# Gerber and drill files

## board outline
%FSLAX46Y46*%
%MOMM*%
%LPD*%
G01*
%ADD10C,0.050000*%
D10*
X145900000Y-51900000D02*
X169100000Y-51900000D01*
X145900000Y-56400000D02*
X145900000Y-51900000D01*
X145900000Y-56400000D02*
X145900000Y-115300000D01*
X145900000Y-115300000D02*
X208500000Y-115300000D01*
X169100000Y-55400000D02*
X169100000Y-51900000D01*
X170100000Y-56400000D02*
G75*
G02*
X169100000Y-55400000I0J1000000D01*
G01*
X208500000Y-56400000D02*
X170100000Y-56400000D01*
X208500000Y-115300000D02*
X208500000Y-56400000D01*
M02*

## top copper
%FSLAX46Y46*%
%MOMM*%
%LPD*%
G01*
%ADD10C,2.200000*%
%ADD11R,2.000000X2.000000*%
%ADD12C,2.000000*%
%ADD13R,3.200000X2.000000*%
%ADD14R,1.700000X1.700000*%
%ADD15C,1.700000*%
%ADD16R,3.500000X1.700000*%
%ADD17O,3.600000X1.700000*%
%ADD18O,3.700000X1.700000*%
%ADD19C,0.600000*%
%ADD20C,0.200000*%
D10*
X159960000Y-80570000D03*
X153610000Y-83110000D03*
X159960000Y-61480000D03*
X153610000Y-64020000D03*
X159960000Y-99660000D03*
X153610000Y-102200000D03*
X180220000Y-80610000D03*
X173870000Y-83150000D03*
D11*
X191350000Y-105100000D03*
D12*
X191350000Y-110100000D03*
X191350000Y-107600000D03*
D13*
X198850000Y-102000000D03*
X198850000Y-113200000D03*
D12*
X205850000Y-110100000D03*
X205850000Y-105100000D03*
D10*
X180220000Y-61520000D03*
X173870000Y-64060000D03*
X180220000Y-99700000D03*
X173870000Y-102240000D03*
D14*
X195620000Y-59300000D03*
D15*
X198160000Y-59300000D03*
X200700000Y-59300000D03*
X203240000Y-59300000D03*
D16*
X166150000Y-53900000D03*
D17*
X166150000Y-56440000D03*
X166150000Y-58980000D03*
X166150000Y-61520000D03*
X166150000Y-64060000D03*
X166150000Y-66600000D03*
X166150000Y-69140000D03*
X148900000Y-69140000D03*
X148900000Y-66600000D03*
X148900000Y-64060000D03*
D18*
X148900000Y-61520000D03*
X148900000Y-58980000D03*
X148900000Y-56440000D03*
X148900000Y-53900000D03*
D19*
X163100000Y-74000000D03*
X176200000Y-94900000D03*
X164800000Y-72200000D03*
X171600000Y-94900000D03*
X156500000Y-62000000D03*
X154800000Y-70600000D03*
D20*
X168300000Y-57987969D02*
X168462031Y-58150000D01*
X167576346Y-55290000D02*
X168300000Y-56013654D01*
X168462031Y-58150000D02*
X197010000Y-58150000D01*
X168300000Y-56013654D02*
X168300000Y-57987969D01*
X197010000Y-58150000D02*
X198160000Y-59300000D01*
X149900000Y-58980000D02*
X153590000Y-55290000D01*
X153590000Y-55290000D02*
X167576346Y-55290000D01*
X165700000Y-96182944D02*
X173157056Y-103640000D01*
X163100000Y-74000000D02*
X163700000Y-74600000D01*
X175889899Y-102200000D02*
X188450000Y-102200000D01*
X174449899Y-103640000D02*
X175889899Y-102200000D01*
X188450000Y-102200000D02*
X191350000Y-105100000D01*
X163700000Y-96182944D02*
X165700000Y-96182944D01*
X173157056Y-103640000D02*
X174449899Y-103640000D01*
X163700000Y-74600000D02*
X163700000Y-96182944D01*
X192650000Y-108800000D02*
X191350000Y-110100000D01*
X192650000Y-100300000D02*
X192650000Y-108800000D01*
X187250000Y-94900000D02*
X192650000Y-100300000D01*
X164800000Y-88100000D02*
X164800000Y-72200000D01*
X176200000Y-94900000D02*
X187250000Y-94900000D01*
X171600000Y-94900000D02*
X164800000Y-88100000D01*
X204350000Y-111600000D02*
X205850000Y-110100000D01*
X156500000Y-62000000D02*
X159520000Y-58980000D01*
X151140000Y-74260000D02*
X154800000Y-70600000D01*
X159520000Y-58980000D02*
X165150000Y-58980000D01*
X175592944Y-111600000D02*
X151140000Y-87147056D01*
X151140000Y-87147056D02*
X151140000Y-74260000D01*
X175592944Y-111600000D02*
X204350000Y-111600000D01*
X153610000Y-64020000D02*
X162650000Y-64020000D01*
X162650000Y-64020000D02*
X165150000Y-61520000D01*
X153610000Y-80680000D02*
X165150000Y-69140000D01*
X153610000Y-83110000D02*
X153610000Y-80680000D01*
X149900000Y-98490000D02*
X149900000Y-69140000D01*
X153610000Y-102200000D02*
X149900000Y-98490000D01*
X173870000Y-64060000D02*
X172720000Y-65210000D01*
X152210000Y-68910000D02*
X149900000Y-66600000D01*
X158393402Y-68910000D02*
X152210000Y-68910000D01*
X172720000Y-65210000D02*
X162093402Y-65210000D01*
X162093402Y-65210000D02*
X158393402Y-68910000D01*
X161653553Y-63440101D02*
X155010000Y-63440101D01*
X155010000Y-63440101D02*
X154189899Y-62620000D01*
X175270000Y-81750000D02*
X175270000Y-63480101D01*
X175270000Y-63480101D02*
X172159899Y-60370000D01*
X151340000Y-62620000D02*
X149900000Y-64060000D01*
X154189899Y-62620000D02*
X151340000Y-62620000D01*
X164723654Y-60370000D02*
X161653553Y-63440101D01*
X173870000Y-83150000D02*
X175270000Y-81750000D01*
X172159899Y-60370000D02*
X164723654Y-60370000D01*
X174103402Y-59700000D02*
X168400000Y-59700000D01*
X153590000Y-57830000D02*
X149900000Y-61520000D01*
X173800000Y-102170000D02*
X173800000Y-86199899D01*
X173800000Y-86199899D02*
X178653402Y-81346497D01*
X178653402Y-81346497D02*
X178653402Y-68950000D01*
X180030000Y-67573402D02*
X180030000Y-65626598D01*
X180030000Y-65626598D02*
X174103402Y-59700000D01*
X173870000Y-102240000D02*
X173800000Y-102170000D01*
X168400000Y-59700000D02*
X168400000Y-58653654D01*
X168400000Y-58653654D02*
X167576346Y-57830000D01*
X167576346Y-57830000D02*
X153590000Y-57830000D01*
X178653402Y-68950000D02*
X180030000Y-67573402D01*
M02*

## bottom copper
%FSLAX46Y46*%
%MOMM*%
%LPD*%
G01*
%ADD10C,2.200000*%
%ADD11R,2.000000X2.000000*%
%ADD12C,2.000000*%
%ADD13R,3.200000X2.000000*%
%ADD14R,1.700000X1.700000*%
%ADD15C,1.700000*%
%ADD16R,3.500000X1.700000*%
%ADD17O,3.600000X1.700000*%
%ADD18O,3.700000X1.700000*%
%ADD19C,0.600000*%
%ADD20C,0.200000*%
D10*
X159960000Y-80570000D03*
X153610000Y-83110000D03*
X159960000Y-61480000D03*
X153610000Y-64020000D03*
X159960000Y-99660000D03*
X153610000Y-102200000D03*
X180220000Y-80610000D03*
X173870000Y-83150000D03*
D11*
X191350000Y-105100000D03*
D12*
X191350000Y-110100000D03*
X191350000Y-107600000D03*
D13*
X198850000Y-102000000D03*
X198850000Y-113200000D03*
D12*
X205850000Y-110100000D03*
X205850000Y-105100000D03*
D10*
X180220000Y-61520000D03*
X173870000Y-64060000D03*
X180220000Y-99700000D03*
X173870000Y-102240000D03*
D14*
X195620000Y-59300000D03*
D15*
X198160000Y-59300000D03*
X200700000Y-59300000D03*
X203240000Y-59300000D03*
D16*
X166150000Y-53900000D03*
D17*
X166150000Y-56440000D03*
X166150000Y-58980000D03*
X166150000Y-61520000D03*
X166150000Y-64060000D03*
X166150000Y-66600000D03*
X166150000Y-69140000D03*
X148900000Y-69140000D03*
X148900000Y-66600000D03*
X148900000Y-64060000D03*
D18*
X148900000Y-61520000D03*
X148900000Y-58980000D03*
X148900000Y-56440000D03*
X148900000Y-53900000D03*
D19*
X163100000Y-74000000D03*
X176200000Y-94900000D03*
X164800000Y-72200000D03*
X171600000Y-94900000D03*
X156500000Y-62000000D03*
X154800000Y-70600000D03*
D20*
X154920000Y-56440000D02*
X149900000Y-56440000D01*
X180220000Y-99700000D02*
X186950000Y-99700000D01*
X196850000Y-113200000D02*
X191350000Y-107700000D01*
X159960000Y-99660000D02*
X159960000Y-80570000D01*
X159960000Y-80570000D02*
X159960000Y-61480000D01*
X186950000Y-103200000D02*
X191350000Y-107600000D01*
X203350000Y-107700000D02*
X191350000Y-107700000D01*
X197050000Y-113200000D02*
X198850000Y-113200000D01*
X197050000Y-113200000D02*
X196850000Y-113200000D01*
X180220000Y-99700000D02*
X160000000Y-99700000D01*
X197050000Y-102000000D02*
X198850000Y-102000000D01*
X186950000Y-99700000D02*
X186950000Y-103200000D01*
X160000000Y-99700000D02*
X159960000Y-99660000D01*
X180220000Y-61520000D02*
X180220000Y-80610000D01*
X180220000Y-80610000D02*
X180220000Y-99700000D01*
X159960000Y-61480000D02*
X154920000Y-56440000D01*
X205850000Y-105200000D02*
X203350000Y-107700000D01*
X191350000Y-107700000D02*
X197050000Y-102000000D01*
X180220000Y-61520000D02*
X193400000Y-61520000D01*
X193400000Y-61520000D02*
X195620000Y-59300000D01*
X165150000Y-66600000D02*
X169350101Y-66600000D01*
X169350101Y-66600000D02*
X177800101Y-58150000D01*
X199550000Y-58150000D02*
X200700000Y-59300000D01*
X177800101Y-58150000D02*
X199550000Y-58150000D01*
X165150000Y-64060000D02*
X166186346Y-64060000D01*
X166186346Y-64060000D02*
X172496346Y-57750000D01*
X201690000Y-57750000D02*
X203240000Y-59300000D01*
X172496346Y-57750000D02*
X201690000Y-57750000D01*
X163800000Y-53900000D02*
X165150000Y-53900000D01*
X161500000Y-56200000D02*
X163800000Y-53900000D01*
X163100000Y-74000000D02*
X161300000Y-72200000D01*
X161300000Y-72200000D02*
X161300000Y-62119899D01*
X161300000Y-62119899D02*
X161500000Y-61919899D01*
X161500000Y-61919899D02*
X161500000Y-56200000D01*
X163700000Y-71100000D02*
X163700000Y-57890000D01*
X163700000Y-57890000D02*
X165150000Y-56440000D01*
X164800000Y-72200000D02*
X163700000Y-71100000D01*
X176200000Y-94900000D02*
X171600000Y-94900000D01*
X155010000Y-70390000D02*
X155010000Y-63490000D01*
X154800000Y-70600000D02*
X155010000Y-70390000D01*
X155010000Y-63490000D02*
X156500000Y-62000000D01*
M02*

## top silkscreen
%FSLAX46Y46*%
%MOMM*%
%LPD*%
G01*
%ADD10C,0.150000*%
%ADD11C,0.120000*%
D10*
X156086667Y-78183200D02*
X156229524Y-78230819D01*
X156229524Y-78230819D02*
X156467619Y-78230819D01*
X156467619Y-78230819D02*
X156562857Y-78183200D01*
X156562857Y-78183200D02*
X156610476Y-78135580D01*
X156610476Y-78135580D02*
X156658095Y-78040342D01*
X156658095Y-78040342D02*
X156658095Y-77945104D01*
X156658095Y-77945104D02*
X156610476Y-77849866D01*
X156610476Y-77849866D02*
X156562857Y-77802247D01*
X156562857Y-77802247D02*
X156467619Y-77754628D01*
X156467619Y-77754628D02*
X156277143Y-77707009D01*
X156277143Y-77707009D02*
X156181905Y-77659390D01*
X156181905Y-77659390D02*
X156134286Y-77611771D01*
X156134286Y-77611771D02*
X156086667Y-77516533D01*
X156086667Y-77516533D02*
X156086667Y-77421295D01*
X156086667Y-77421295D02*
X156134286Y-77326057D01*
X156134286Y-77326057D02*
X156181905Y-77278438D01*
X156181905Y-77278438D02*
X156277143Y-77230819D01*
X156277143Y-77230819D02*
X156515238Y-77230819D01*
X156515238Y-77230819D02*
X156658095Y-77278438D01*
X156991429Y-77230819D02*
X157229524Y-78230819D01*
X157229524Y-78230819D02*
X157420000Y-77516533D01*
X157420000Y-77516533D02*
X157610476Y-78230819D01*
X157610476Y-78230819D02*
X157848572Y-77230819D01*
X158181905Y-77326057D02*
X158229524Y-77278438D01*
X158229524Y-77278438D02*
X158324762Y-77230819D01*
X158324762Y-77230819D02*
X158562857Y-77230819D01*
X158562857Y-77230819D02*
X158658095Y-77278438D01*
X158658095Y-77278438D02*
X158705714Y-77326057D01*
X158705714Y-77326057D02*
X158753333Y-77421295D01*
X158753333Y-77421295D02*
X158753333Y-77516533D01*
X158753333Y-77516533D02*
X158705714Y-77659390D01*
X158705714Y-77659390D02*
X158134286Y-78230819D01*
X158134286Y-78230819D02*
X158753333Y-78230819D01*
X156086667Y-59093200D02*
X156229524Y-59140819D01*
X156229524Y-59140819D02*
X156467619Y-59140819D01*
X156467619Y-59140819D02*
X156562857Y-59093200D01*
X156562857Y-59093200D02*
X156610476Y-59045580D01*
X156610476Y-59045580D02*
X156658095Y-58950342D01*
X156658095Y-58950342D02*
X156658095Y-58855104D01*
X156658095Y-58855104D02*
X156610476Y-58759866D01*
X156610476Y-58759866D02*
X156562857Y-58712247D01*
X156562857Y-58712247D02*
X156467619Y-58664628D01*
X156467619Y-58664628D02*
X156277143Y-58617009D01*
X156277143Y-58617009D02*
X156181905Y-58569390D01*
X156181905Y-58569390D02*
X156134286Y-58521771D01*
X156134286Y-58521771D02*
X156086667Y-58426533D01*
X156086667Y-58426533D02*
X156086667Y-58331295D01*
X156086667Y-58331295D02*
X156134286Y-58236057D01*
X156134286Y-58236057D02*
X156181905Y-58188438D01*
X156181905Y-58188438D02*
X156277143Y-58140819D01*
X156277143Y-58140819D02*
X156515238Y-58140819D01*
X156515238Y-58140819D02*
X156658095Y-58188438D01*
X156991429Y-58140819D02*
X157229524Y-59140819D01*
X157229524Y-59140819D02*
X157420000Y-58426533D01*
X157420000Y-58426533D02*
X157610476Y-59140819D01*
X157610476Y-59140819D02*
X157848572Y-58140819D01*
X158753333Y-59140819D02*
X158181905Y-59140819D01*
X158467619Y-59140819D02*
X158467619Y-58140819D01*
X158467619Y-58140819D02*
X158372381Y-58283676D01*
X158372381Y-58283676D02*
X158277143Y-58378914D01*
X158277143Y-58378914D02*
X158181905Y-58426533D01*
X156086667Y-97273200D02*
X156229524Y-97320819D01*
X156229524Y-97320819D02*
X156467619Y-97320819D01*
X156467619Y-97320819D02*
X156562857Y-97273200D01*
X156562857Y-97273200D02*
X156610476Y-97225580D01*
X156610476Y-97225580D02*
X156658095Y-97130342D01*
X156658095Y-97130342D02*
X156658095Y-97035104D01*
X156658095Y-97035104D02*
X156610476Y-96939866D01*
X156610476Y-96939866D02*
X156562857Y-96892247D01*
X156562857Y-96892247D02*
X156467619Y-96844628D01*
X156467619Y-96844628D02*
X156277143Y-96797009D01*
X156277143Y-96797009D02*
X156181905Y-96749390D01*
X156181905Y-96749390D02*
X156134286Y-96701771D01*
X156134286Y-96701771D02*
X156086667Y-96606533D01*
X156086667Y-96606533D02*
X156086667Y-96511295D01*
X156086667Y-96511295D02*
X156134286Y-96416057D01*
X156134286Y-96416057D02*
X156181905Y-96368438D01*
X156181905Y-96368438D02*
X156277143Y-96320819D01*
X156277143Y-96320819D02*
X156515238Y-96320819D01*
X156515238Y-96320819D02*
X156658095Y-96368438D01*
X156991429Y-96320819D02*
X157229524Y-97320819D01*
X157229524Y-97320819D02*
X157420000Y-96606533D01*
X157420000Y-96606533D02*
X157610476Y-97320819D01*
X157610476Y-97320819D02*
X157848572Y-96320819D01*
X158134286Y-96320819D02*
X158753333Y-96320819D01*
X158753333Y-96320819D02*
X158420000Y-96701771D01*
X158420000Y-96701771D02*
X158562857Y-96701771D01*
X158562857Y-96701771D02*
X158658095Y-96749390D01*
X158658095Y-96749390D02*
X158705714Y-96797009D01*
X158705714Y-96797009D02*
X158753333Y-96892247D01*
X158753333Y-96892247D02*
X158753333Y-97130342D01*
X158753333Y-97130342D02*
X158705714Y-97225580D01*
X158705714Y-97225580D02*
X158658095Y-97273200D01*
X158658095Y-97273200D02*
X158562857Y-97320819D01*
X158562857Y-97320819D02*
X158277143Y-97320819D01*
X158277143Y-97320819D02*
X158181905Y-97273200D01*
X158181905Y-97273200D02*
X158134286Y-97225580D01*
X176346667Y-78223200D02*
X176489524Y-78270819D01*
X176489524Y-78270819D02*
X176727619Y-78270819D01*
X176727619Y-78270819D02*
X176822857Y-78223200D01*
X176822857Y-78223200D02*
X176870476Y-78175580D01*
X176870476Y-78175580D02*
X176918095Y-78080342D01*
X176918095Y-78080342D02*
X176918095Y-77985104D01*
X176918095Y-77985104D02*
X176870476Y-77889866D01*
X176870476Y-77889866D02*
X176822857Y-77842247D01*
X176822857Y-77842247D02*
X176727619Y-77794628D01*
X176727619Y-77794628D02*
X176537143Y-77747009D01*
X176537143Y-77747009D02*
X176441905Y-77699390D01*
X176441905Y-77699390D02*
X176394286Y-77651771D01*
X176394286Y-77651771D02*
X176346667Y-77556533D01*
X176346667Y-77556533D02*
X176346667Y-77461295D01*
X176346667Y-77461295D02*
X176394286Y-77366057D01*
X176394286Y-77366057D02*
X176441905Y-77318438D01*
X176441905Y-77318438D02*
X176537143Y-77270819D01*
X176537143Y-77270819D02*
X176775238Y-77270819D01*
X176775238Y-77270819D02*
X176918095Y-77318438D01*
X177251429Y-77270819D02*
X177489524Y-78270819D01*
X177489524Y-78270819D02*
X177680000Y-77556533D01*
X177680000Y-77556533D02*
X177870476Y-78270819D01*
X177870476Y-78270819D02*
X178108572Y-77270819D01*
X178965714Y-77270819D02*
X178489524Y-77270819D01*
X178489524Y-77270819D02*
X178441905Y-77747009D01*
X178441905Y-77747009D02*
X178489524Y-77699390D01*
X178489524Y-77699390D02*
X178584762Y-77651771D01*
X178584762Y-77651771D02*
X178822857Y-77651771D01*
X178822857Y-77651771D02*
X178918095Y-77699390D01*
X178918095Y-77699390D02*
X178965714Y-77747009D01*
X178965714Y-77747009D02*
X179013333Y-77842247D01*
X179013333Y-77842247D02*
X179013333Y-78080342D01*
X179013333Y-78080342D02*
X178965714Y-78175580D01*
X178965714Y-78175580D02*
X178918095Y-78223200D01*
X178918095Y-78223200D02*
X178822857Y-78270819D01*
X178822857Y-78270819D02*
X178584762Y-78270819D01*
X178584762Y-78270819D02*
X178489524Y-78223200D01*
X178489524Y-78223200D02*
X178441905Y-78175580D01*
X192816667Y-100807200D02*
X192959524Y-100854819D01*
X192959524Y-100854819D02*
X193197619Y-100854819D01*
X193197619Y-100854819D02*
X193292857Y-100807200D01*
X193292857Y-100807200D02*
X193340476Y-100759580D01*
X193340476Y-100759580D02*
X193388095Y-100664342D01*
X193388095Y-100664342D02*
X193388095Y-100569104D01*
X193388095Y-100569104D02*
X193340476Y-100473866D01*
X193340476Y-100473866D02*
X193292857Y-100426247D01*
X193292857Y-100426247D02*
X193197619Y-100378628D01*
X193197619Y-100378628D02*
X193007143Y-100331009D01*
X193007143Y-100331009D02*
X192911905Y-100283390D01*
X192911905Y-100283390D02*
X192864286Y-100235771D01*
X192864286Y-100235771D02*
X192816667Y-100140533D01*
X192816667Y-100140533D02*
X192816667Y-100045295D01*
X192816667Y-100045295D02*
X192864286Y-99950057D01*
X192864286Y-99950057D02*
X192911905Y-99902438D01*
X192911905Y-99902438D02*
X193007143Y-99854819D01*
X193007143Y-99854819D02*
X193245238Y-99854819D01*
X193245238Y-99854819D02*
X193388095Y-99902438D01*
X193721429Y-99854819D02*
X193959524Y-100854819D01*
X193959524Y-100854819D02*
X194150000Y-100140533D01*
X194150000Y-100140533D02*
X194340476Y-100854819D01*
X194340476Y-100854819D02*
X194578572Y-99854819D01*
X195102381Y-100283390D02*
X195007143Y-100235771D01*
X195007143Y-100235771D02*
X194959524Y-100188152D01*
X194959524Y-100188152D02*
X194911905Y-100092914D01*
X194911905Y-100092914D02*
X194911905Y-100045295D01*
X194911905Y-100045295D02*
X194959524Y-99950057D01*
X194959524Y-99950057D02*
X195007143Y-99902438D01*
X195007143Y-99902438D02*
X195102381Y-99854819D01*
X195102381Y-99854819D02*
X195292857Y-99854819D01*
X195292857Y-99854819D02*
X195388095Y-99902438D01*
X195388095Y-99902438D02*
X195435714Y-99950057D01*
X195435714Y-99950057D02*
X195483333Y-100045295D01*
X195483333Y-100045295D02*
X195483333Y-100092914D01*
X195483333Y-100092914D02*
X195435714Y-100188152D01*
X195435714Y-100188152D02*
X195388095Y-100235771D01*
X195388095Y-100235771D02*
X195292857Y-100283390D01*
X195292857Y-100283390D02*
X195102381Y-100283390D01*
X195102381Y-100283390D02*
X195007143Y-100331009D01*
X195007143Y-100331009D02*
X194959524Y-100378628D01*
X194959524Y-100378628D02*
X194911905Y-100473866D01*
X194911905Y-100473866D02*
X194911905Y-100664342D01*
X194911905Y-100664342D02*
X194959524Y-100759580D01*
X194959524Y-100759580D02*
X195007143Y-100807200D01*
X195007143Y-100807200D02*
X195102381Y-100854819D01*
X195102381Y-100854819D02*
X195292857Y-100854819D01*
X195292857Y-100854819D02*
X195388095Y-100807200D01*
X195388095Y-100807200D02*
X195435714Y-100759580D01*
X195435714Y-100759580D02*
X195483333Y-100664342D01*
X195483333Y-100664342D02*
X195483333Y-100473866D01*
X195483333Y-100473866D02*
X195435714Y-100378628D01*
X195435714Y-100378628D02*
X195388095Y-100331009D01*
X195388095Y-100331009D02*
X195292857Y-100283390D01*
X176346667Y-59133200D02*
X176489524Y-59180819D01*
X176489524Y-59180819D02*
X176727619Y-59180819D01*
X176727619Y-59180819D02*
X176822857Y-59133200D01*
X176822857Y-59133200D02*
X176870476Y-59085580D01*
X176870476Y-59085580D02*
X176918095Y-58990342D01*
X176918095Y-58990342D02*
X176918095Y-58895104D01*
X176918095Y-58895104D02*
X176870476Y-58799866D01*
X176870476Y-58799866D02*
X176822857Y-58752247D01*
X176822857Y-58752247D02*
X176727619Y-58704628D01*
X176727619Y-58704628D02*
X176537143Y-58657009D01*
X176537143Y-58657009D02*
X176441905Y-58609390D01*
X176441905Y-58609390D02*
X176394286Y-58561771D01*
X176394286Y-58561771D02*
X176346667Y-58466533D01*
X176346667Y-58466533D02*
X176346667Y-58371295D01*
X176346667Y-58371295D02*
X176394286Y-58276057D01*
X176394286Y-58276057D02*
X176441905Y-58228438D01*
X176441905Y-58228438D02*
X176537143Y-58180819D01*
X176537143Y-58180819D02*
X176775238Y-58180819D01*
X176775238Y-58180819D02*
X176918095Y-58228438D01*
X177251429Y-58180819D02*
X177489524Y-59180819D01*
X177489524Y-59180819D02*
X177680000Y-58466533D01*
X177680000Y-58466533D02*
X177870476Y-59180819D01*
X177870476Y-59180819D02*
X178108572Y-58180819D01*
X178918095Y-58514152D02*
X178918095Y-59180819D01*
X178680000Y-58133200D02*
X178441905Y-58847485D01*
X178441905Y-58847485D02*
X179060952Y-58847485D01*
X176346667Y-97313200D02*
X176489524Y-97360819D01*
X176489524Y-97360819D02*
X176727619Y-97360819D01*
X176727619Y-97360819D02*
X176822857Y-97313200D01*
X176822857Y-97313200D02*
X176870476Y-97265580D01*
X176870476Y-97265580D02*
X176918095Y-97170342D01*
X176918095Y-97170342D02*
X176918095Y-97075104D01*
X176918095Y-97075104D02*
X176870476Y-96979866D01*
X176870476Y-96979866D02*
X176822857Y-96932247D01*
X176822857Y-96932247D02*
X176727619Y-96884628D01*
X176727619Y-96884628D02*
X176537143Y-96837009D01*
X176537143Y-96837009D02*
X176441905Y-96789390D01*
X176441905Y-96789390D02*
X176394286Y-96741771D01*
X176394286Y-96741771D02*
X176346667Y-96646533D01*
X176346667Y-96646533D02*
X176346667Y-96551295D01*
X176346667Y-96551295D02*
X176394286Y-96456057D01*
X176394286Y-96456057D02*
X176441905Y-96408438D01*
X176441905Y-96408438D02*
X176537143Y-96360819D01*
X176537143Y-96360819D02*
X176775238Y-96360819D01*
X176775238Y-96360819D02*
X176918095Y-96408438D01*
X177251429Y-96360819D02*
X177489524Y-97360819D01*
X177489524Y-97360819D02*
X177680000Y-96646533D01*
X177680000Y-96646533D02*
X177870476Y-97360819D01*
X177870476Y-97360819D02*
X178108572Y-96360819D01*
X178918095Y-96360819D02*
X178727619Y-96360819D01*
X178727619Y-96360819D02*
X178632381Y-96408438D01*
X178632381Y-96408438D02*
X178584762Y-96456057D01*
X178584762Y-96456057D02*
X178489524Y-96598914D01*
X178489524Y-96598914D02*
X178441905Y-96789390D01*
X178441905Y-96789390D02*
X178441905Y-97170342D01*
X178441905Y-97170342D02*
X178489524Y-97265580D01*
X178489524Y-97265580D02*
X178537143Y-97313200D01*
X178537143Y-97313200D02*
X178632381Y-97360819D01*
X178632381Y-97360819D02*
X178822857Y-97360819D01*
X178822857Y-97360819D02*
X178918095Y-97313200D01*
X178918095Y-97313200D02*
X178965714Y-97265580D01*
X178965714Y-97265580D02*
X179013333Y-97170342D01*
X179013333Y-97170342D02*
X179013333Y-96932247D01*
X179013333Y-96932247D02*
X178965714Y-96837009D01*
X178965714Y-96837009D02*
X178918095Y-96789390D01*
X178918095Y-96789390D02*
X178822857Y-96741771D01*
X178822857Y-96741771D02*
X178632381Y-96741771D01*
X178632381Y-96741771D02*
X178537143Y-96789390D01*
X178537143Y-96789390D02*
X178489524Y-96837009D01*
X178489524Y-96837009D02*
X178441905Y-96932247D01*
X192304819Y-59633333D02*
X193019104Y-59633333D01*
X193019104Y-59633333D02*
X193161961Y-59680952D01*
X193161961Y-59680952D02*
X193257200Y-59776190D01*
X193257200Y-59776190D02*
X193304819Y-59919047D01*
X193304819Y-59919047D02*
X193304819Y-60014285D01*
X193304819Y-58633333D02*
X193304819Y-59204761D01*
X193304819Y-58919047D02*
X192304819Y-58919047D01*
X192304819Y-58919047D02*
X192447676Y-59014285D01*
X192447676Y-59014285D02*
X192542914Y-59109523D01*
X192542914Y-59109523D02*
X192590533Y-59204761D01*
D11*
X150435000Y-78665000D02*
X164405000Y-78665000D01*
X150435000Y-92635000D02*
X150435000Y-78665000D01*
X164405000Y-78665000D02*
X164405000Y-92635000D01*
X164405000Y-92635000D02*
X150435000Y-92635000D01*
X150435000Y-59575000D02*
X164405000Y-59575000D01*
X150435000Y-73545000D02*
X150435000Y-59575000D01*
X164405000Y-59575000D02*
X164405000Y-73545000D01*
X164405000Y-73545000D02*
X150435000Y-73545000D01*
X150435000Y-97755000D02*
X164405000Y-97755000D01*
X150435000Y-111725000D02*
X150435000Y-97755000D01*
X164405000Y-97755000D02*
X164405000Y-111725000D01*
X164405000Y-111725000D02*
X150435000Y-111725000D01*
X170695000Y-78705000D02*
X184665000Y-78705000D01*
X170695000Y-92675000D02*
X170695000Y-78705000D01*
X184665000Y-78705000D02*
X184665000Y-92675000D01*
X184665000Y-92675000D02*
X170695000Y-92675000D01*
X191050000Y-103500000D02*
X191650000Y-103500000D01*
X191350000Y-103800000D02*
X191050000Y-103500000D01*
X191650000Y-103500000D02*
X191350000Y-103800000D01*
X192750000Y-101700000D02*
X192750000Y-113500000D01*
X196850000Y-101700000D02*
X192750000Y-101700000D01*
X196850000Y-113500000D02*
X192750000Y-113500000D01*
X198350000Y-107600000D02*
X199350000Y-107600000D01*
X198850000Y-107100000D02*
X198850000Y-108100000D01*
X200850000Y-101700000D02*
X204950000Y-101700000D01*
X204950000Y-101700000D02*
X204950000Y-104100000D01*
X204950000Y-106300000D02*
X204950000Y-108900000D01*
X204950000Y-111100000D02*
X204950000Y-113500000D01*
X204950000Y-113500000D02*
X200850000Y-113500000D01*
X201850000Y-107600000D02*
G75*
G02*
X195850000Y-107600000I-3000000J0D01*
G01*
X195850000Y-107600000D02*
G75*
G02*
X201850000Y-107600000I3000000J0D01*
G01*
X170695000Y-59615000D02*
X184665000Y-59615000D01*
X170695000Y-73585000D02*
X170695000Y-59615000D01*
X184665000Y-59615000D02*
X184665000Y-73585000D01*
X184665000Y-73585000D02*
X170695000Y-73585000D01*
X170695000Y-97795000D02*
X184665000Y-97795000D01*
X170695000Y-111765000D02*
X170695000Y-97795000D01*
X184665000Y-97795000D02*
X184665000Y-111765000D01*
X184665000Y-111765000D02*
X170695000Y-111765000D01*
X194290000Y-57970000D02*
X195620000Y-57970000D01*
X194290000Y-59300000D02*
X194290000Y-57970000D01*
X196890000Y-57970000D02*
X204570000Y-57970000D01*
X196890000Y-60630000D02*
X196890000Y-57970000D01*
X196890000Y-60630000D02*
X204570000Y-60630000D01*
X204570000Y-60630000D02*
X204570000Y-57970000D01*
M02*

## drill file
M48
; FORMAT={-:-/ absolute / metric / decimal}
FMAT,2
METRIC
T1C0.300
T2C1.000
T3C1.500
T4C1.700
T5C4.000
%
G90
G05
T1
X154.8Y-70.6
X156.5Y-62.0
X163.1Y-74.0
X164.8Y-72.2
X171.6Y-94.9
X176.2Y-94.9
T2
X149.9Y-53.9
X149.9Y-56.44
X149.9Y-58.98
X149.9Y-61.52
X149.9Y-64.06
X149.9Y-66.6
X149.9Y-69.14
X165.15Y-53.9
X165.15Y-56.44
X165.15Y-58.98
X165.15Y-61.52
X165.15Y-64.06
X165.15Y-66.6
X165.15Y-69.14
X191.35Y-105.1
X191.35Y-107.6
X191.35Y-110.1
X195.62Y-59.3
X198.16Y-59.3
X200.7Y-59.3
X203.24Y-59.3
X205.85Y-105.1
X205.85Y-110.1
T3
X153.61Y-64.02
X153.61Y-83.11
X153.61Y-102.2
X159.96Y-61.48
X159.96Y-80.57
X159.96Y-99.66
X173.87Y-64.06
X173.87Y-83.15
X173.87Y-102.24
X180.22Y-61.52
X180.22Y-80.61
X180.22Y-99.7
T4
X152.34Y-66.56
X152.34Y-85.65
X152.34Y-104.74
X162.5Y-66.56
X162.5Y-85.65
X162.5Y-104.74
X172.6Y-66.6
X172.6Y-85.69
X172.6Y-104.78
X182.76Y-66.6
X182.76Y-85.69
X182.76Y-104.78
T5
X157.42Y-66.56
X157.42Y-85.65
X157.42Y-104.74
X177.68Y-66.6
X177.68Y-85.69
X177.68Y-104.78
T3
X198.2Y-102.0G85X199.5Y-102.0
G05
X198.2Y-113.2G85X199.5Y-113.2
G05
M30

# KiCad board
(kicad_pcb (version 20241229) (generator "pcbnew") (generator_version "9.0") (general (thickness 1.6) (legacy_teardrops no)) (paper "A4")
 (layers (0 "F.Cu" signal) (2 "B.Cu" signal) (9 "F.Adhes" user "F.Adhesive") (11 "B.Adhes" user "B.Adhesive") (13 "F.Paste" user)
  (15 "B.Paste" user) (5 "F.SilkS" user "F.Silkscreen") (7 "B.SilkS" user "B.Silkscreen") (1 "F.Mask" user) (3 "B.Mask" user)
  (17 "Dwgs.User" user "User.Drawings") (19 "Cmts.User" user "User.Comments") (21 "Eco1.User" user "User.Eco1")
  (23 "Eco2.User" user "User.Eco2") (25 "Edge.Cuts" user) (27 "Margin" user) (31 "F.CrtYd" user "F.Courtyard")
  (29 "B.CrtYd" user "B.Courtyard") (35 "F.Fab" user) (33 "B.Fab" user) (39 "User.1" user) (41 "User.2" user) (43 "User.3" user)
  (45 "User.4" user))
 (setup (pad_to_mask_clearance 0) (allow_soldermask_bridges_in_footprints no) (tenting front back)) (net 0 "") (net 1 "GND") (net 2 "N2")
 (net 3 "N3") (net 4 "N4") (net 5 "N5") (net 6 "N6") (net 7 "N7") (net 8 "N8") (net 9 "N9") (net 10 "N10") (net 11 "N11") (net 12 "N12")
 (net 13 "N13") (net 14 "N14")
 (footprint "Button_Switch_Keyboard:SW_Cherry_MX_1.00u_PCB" (layer "F.Cu") (at 159.96 80.57)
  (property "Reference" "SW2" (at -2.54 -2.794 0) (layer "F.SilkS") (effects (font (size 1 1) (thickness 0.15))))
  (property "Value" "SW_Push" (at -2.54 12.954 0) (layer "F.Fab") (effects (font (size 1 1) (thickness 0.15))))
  (fp_line (start -9.525 -1.905) (end 4.445 -1.905) (stroke (width 0.12) (type solid)) (layer "F.SilkS"))
  (fp_line (start -9.525 12.065) (end -9.525 -1.905) (stroke (width 0.12) (type solid)) (layer "F.SilkS"))
  (fp_line (start 4.445 -1.905) (end 4.445 12.065) (stroke (width 0.12) (type solid)) (layer "F.SilkS"))
  (fp_line (start 4.445 12.065) (end -9.525 12.065) (stroke (width 0.12) (type solid)) (layer "F.SilkS"))
  (pad "" np_thru_hole circle (at -7.62 5.08) (size 1.7 1.7) (drill 1.7) (layers "*.Cu" "*.Mask"))
  (pad "" np_thru_hole circle (at -2.54 5.08) (size 4 4) (drill 4) (layers "*.Cu" "*.Mask"))
  (pad "" np_thru_hole circle (at 2.54 5.08) (size 1.7 1.7) (drill 1.7) (layers "*.Cu" "*.Mask"))
  (pad "1" thru_hole circle (at 0 0) (size 2.2 2.2) (drill 1.5) (layers "*.Cu" "*.Mask") (remove_unused_layers no) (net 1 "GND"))
  (pad "2" thru_hole circle (at -6.35 2.54) (size 2.2 2.2) (drill 1.5) (layers "*.Cu" "*.Mask") (remove_unused_layers no) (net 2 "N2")))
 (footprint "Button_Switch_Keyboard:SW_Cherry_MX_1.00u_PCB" (layer "F.Cu") (at 159.96 61.48)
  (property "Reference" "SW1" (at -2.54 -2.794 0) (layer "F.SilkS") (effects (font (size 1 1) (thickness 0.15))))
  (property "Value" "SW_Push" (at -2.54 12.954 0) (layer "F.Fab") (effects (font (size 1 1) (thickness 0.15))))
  (fp_line (start -9.525 -1.905) (end 4.445 -1.905) (stroke (width 0.12) (type solid)) (layer "F.SilkS"))
  (fp_line (start -9.525 12.065) (end -9.525 -1.905) (stroke (width 0.12) (type solid)) (layer "F.SilkS"))
  (fp_line (start 4.445 -1.905) (end 4.445 12.065) (stroke (width 0.12) (type solid)) (layer "F.SilkS"))
  (fp_line (start 4.445 12.065) (end -9.525 12.065) (stroke (width 0.12) (type solid)) (layer "F.SilkS"))
  (pad "" np_thru_hole circle (at -7.62 5.08) (size 1.7 1.7) (drill 1.7) (layers "*.Cu" "*.Mask"))
  (pad "" np_thru_hole circle (at -2.54 5.08) (size 4 4) (drill 4) (layers "*.Cu" "*.Mask"))
  (pad "" np_thru_hole circle (at 2.54 5.08) (size 1.7 1.7) (drill 1.7) (layers "*.Cu" "*.Mask"))
  (pad "1" thru_hole circle (at 0 0) (size 2.2 2.2) (drill 1.5) (layers "*.Cu" "*.Mask") (remove_unused_layers no) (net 1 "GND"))
  (pad "2" thru_hole circle (at -6.35 2.54) (size 2.2 2.2) (drill 1.5) (layers "*.Cu" "*.Mask") (remove_unused_layers no) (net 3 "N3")))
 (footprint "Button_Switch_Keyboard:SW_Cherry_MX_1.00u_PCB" (layer "F.Cu") (at 159.96 99.66)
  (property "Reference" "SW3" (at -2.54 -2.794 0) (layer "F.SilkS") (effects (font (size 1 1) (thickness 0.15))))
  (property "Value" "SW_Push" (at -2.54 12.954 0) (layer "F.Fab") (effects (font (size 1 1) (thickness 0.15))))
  (fp_line (start -9.525 -1.905) (end 4.445 -1.905) (stroke (width 0.12) (type solid)) (layer "F.SilkS"))
  (fp_line (start -9.525 12.065) (end -9.525 -1.905) (stroke (width 0.12) (type solid)) (layer "F.SilkS"))
  (fp_line (start 4.445 -1.905) (end 4.445 12.065) (stroke (width 0.12) (type solid)) (layer "F.SilkS"))
  (fp_line (start 4.445 12.065) (end -9.525 12.065) (stroke (width 0.12) (type solid)) (layer "F.SilkS"))
  (pad "" np_thru_hole circle (at -7.62 5.08) (size 1.7 1.7) (drill 1.7) (layers "*.Cu" "*.Mask"))
  (pad "" np_thru_hole circle (at -2.54 5.08) (size 4 4) (drill 4) (layers "*.Cu" "*.Mask"))
  (pad "" np_thru_hole circle (at 2.54 5.08) (size 1.7 1.7) (drill 1.7) (layers "*.Cu" "*.Mask"))
  (pad "1" thru_hole circle (at 0 0) (size 2.2 2.2) (drill 1.5) (layers "*.Cu" "*.Mask") (remove_unused_layers no) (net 1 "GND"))
  (pad "2" thru_hole circle (at -6.35 2.54) (size 2.2 2.2) (drill 1.5) (layers "*.Cu" "*.Mask") (remove_unused_layers no) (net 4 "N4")))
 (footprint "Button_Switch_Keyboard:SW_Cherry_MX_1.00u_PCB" (layer "F.Cu") (at 180.22 80.61)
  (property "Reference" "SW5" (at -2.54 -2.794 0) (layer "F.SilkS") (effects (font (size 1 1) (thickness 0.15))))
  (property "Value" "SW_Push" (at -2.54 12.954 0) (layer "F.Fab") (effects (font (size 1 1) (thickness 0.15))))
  (fp_line (start -9.525 -1.905) (end 4.445 -1.905) (stroke (width 0.12) (type solid)) (layer "F.SilkS"))
  (fp_line (start -9.525 12.065) (end -9.525 -1.905) (stroke (width 0.12) (type solid)) (layer "F.SilkS"))
  (fp_line (start 4.445 -1.905) (end 4.445 12.065) (stroke (width 0.12) (type solid)) (layer "F.SilkS"))
  (fp_line (start 4.445 12.065) (end -9.525 12.065) (stroke (width 0.12) (type solid)) (layer "F.SilkS"))
  (pad "" np_thru_hole circle (at -7.62 5.08) (size 1.7 1.7) (drill 1.7) (layers "*.Cu" "*.Mask"))
  (pad "" np_thru_hole circle (at -2.54 5.08) (size 4 4) (drill 4) (layers "*.Cu" "*.Mask"))
  (pad "" np_thru_hole circle (at 2.54 5.08) (size 1.7 1.7) (drill 1.7) (layers "*.Cu" "*.Mask"))
  (pad "1" thru_hole circle (at 0 0) (size 2.2 2.2) (drill 1.5) (layers "*.Cu" "*.Mask") (remove_unused_layers no) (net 1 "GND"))
  (pad "2" thru_hole circle (at -6.35 2.54) (size 2.2 2.2) (drill 1.5) (layers "*.Cu" "*.Mask") (remove_unused_layers no) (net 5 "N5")))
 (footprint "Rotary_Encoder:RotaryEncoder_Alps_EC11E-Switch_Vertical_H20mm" (layer "F.Cu") (at 191.35 105.1)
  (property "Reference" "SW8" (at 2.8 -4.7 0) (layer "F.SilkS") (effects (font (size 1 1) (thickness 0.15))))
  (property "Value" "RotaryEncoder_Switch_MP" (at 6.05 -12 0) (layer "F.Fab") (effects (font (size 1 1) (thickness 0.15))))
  (fp_line (start -0.3 -1.6) (end 0.3 -1.6) (stroke (width 0.12) (type solid)) (layer "F.SilkS"))
  (fp_line (start 0 -1.3) (end -0.3 -1.6) (stroke (width 0.12) (type solid)) (layer "F.SilkS"))
  (fp_line (start 0.3 -1.6) (end 0 -1.3) (stroke (width 0.12) (type solid)) (layer "F.SilkS"))
  (fp_line (start 1.4 -3.4) (end 1.4 8.4) (stroke (width 0.12) (type solid)) (layer "F.SilkS"))
  (fp_line (start 5.5 -3.4) (end 1.4 -3.4) (stroke (width 0.12) (type solid)) (layer "F.SilkS"))
  (fp_line (start 5.5 8.4) (end 1.4 8.4) (stroke (width 0.12) (type solid)) (layer "F.SilkS"))
  (fp_line (start 7 2.5) (end 8 2.5) (stroke (width 0.12) (type solid)) (layer "F.SilkS"))
  (fp_line (start 7.5 2) (end 7.5 3) (stroke (width 0.12) (type solid)) (layer "F.SilkS"))
  (fp_line (start 9.5 -3.4) (end 13.6 -3.4) (stroke (width 0.12) (type solid)) (layer "F.SilkS"))
  (fp_line (start 13.6 -3.4) (end 13.6 -1) (stroke (width 0.12) (type solid)) (layer "F.SilkS"))
  (fp_line (start 13.6 1.2) (end 13.6 3.8) (stroke (width 0.12) (type solid)) (layer "F.SilkS"))
  (fp_line (start 13.6 6) (end 13.6 8.4) (stroke (width 0.12) (type solid)) (layer "F.SilkS"))
  (fp_line (start 13.6 8.4) (end 9.5 8.4) (stroke (width 0.12) (type solid)) (layer "F.SilkS"))
  (fp_circle (center 7.5 2.5) (end 10.5 2.5) (stroke (width 0.12) (type solid)) (fill no) (layer "F.SilkS"))
  (pad "A" thru_hole rect (at 0 0) (size 2 2) (drill 1) (layers "*.Cu" "*.Mask") (remove_unused_layers no) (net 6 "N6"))
  (pad "B" thru_hole circle (at 0 5) (size 2 2) (drill 1) (layers "*.Cu" "*.Mask") (remove_unused_layers no) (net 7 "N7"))
  (pad "C" thru_hole circle (at 0 2.5) (size 2 2) (drill 1) (layers "*.Cu" "*.Mask") (remove_unused_layers no) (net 1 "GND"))
  (pad "MP" thru_hole rect (at 7.5 -3.1) (size 3.2 2) (drill oval 2.8 1.5) (layers "*.Cu" "*.Mask") (remove_unused_layers no) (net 1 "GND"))
  (pad "MP" thru_hole rect (at 7.5 8.1) (size 3.2 2) (drill oval 2.8 1.5) (layers "*.Cu" "*.Mask") (remove_unused_layers no) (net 1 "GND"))
  (pad "S1" thru_hole circle (at 14.5 5) (size 2 2) (drill 1) (layers "*.Cu" "*.Mask") (remove_unused_layers no) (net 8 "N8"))
  (pad "S2" thru_hole circle (at 14.5 0) (size 2 2) (drill 1) (layers "*.Cu" "*.Mask") (remove_unused_layers no) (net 1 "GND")))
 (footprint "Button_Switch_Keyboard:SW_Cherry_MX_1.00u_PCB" (layer "F.Cu") (at 180.22 61.52)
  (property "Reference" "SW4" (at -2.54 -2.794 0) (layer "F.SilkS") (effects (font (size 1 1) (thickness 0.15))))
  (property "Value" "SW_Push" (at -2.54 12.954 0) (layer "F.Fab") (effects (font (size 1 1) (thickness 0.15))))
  (fp_line (start -9.525 -1.905) (end 4.445 -1.905) (stroke (width 0.12) (type solid)) (layer "F.SilkS"))
  (fp_line (start -9.525 12.065) (end -9.525 -1.905) (stroke (width 0.12) (type solid)) (layer "F.SilkS"))
  (fp_line (start 4.445 -1.905) (end 4.445 12.065) (stroke (width 0.12) (type solid)) (layer "F.SilkS"))
  (fp_line (start 4.445 12.065) (end -9.525 12.065) (stroke (width 0.12) (type solid)) (layer "F.SilkS"))
  (pad "" np_thru_hole circle (at -7.62 5.08) (size 1.7 1.7) (drill 1.7) (layers "*.Cu" "*.Mask"))
  (pad "" np_thru_hole circle (at -2.54 5.08) (size 4 4) (drill 4) (layers "*.Cu" "*.Mask"))
  (pad "" np_thru_hole circle (at 2.54 5.08) (size 1.7 1.7) (drill 1.7) (layers "*.Cu" "*.Mask"))
  (pad "1" thru_hole circle (at 0 0) (size 2.2 2.2) (drill 1.5) (layers "*.Cu" "*.Mask") (remove_unused_layers no) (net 1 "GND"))
  (pad "2" thru_hole circle (at -6.35 2.54) (size 2.2 2.2) (drill 1.5) (layers "*.Cu" "*.Mask") (remove_unused_layers no) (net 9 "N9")))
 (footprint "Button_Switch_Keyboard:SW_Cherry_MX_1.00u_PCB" (layer "F.Cu") (at 180.22 99.7)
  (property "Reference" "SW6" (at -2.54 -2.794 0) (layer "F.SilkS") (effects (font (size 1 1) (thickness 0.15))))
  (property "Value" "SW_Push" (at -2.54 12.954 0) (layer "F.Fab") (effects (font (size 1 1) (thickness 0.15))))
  (fp_line (start -9.525 -1.905) (end 4.445 -1.905) (stroke (width 0.12) (type solid)) (layer "F.SilkS"))
  (fp_line (start -9.525 12.065) (end -9.525 -1.905) (stroke (width 0.12) (type solid)) (layer "F.SilkS"))
  (fp_line (start 4.445 -1.905) (end 4.445 12.065) (stroke (width 0.12) (type solid)) (layer "F.SilkS"))
  (fp_line (start 4.445 12.065) (end -9.525 12.065) (stroke (width 0.12) (type solid)) (layer "F.SilkS"))
  (pad "" np_thru_hole circle (at -7.62 5.08) (size 1.7 1.7) (drill 1.7) (layers "*.Cu" "*.Mask"))
  (pad "" np_thru_hole circle (at -2.54 5.08) (size 4 4) (drill 4) (layers "*.Cu" "*.Mask"))
  (pad "" np_thru_hole circle (at 2.54 5.08) (size 1.7 1.7) (drill 1.7) (layers "*.Cu" "*.Mask"))
  (pad "1" thru_hole circle (at 0 0) (size 2.2 2.2) (drill 1.5) (layers "*.Cu" "*.Mask") (remove_unused_layers no) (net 1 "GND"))
  (pad "2" thru_hole circle (at -6.35 2.54) (size 2.2 2.2) (drill 1.5) (layers "*.Cu" "*.Mask") (remove_unused_layers no) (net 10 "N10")))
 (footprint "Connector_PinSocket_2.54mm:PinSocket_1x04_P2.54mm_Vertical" (layer "F.Cu") (at 195.62 59.3 90)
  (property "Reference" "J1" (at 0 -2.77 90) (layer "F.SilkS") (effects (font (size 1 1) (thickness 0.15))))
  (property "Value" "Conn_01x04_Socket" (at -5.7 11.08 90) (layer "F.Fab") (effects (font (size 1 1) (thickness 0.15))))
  (fp_line (start 1.33 -1.33) (end 1.33 0) (stroke (width 0.12) (type solid)) (layer "F.SilkS"))
  (fp_line (start 0 -1.33) (end 1.33 -1.33) (stroke (width 0.12) (type solid)) (layer "F.SilkS"))
  (fp_line (start 1.33 1.27) (end 1.33 8.95) (stroke (width 0.12) (type solid)) (layer "F.SilkS"))
  (fp_line (start -1.33 1.27) (end 1.33 1.27) (stroke (width 0.12) (type solid)) (layer "F.SilkS"))
  (fp_line (start -1.33 1.27) (end -1.33 8.95) (stroke (width 0.12) (type solid)) (layer "F.SilkS"))
  (fp_line (start -1.33 8.95) (end 1.33 8.95) (stroke (width 0.12) (type solid)) (layer "F.SilkS"))
  (pad "1" thru_hole rect (at 0 0 90) (size 1.7 1.7) (drill 1) (layers "*.Cu" "*.Mask") (remove_unused_layers no) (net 1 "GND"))
  (pad "2" thru_hole circle (at 0 2.54 90) (size 1.7 1.7) (drill 1) (layers "*.Cu" "*.Mask") (remove_unused_layers no) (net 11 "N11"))
  (pad "3" thru_hole circle (at 0 5.08 90) (size 1.7 1.7) (drill 1) (layers "*.Cu" "*.Mask") (remove_unused_layers no) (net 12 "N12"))
  (pad "4" thru_hole circle (at 0 7.62 90) (size 1.7 1.7) (drill 1) (layers "*.Cu" "*.Mask") (remove_unused_layers no) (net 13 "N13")))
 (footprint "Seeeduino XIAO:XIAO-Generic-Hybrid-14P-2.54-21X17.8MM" (layer "B.Cu") (at 157.525 61.52 180)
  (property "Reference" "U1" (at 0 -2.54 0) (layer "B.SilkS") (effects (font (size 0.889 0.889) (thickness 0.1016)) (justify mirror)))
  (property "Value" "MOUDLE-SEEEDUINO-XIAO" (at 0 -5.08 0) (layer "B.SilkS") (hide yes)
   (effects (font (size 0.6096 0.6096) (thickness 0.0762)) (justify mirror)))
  (pad "1" thru_hole rect (at -7.625 7.62 180) (size 3.5 1.7) (drill 1 (offset -1 0)) (layers "*.Cu" "*.Mask") (remove_unused_layers no)
   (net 6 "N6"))
  (pad "2" thru_hole oval (at -7.625 5.08 180) (size 3.6 1.7) (drill 1 (offset -1 0)) (layers "*.Cu" "*.Mask") (remove_unused_layers no)
   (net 7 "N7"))
  (pad "3" thru_hole oval (at -7.625 2.54 180) (size 3.6 1.7) (drill 1 (offset -1 0)) (layers "*.Cu" "*.Mask") (remove_unused_layers no)
   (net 8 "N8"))
  (pad "4" thru_hole oval (at -7.625 0 180) (size 3.6 1.7) (drill 1 (offset -1 0)) (layers "*.Cu" "*.Mask") (remove_unused_layers no)
   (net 3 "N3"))
  (pad "5" thru_hole oval (at -7.625 -2.54 180) (size 3.6 1.7) (drill 1 (offset -1 0)) (layers "*.Cu" "*.Mask") (remove_unused_layers no)
   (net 13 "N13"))
  (pad "6" thru_hole oval (at -7.625 -5.08) (size 3.6 1.7) (drill 1 (offset 1 0)) (layers "*.Cu" "*.Mask") (remove_unused_layers no)
   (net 12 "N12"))
  (pad "7" thru_hole oval (at -7.625 -7.62 180) (size 3.6 1.7) (drill 1 (offset -1 0)) (layers "*.Cu" "*.Mask") (remove_unused_layers no)
   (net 2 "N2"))
  (pad "8" thru_hole oval (at 7.625 -7.62 180) (size 3.6 1.7) (drill 1 (offset 1 0)) (layers "*.Cu" "*.Mask") (remove_unused_layers no)
   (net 4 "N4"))
  (pad "9" thru_hole oval (at 7.625 -5.08 180) (size 3.6 1.7) (drill 1 (offset 1 0)) (layers "*.Cu" "*.Mask") (remove_unused_layers no)
   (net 9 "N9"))
  (pad "10" thru_hole oval (at 7.625 -2.54 180) (size 3.6 1.7) (drill 1 (offset 1 0)) (layers "*.Cu" "*.Mask") (remove_unused_layers no)
   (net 5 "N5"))
  (pad "11" thru_hole oval (at 7.625 0 180) (size 3.7 1.7) (drill 1 (offset 1 0)) (layers "*.Cu" "*.Mask") (remove_unused_layers no)
   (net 10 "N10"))
  (pad "12" thru_hole oval (at 7.625 2.54 180) (size 3.7 1.7) (drill 1 (offset 1 0)) (layers "*.Cu" "*.Mask") (remove_unused_layers no)
   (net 11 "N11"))
  (pad "13" thru_hole oval (at 7.625 5.08 180) (size 3.7 1.7) (drill 1 (offset 1 0)) (layers "*.Cu" "*.Mask") (remove_unused_layers no)
   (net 1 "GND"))
  (pad "14" thru_hole oval (at 7.625 7.62 180) (size 3.7 1.7) (drill 1 (offset 1 0)) (layers "*.Cu" "*.Mask") (remove_unused_layers no)
   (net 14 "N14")))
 (gr_line (start 145.9 51.9) (end 169.1 51.9) (stroke (width 0.05) (type default)) (layer "Edge.Cuts"))
 (gr_line (start 145.9 56.4) (end 145.9 51.9) (stroke (width 0.05) (type default)) (layer "Edge.Cuts"))
 (gr_line (start 145.9 56.4) (end 145.9 115.3) (stroke (width 0.05) (type default)) (layer "Edge.Cuts"))
 (gr_line (start 145.9 115.3) (end 208.5 115.3) (stroke (width 0.05) (type default)) (layer "Edge.Cuts"))
 (gr_line (start 169.1 55.4) (end 169.1 51.9) (stroke (width 0.05) (type default)) (layer "Edge.Cuts"))
 (gr_arc (start 170.1 56.4) (mid 169.392893 56.107107) (end 169.1 55.4) (stroke (width 0.05) (type default)) (layer "Edge.Cuts"))
 (gr_line (start 208.5 56.4) (end 170.1 56.4) (stroke (width 0.05) (type default)) (layer "Edge.Cuts"))
 (gr_line (start 208.5 115.3) (end 208.5 56.4) (stroke (width 0.05) (type default)) (layer "Edge.Cuts"))
 (segment (start 154.92 56.44) (end 149.9 56.44) (width 0.2) (layer "B.Cu") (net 1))
 (segment (start 180.22 99.7) (end 186.95 99.7) (width 0.2) (layer "B.Cu") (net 1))
 (segment (start 196.85 113.2) (end 191.35 107.7) (width 0.2) (layer "B.Cu") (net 1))
 (segment (start 159.96 99.66) (end 159.96 80.57) (width 0.2) (layer "B.Cu") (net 1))
 (segment (start 159.96 80.57) (end 159.96 61.48) (width 0.2) (layer "B.Cu") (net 1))
 (segment (start 186.95 103.2) (end 191.35 107.6) (width 0.2) (layer "B.Cu") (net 1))
 (segment (start 203.35 107.7) (end 191.35 107.7) (width 0.2) (layer "B.Cu") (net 1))
 (segment (start 197.05 113.2) (end 198.85 113.2) (width 0.2) (layer "B.Cu") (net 1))
 (segment (start 197.05 113.2) (end 196.85 113.2) (width 0.2) (layer "B.Cu") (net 1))
 (segment (start 180.22 99.7) (end 160 99.7) (width 0.2) (layer "B.Cu") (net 1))
 (segment (start 197.05 102) (end 198.85 102) (width 0.2) (layer "B.Cu") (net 1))
 (segment (start 186.95 99.7) (end 186.95 103.2) (width 0.2) (layer "B.Cu") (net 1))
 (segment (start 160 99.7) (end 159.96 99.66) (width 0.2) (layer "B.Cu") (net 1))
 (segment (start 180.22 61.52) (end 180.22 80.61) (width 0.2) (layer "B.Cu") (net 1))
 (segment (start 180.22 80.61) (end 180.22 99.7) (width 0.2) (layer "B.Cu") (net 1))
 (segment (start 159.96 61.48) (end 154.92 56.44) (width 0.2) (layer "B.Cu") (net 1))
 (segment (start 205.85 105.2) (end 203.35 107.7) (width 0.2) (layer "B.Cu") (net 1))
 (segment (start 191.35 107.7) (end 197.05 102) (width 0.2) (layer "B.Cu") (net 1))
 (segment (start 180.22 61.52) (end 193.4 61.52) (width 0.2) (layer "B.Cu") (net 1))
 (segment (start 193.4 61.52) (end 195.62 59.3) (width 0.2) (layer "B.Cu") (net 1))
 (segment (start 165.15 66.6) (end 169.350101 66.6) (width 0.2) (layer "B.Cu") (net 12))
 (segment (start 169.350101 66.6) (end 177.800101 58.15) (width 0.2) (layer "B.Cu") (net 12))
 (segment (start 199.55 58.15) (end 200.7 59.3) (width 0.2) (layer "B.Cu") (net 12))
 (segment (start 177.800101 58.15) (end 199.55 58.15) (width 0.2) (layer "B.Cu") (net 12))
 (segment (start 168.3 57.987969) (end 168.462031 58.15) (width 0.2) (layer "F.Cu") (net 11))
 (segment (start 167.576346 55.29) (end 168.3 56.013654) (width 0.2) (layer "F.Cu") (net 11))
 (segment (start 168.462031 58.15) (end 197.01 58.15) (width 0.2) (layer "F.Cu") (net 11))
 (segment (start 168.3 56.013654) (end 168.3 57.987969) (width 0.2) (layer "F.Cu") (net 11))
 (segment (start 197.01 58.15) (end 198.16 59.3) (width 0.2) (layer "F.Cu") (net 11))
 (segment (start 149.9 58.98) (end 153.59 55.29) (width 0.2) (layer "F.Cu") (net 11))
 (segment (start 153.59 55.29) (end 167.576346 55.29) (width 0.2) (layer "F.Cu") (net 11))
 (segment (start 165.15 64.06) (end 166.186346 64.06) (width 0.2) (layer "B.Cu") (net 13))
 (segment (start 166.186346 64.06) (end 172.496346 57.75) (width 0.2) (layer "B.Cu") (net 13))
 (segment (start 201.69 57.75) (end 203.24 59.3) (width 0.2) (layer "B.Cu") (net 13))
 (segment (start 172.496346 57.75) (end 201.69 57.75) (width 0.2) (layer "B.Cu") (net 13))
 (segment (start 165.7 96.182944) (end 173.157056 103.64) (width 0.2) (layer "F.Cu") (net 6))
 (segment (start 163.1 74) (end 163.7 74.6) (width 0.2) (layer "F.Cu") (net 6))
 (segment (start 175.889899 102.2) (end 188.45 102.2) (width 0.2) (layer "F.Cu") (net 6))
 (segment (start 174.449899 103.64) (end 175.889899 102.2) (width 0.2) (layer "F.Cu") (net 6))
 (segment (start 188.45 102.2) (end 191.35 105.1) (width 0.2) (layer "F.Cu") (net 6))
 (segment (start 163.7 96.182944) (end 165.7 96.182944) (width 0.2) (layer "F.Cu") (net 6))
 (segment (start 173.157056 103.64) (end 174.449899 103.64) (width 0.2) (layer "F.Cu") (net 6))
 (segment (start 163.7 74.6) (end 163.7 96.182944) (width 0.2) (layer "F.Cu") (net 6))
 (via (at 163.1 74) (size 0.6) (drill 0.3) (layers "F.Cu" "B.Cu") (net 6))
 (segment (start 163.8 53.9) (end 165.15 53.9) (width 0.2) (layer "B.Cu") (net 6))
 (segment (start 161.5 56.2) (end 163.8 53.9) (width 0.2) (layer "B.Cu") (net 6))
 (segment (start 163.1 74) (end 161.3 72.2) (width 0.2) (layer "B.Cu") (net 6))
 (segment (start 161.3 72.2) (end 161.3 62.119899) (width 0.2) (layer "B.Cu") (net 6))
 (segment (start 161.3 62.119899) (end 161.5 61.919899) (width 0.2) (layer "B.Cu") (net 6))
 (segment (start 161.5 61.919899) (end 161.5 56.2) (width 0.2) (layer "B.Cu") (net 6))
 (segment (start 192.65 108.8) (end 191.35 110.1) (width 0.2) (layer "F.Cu") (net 7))
 (segment (start 192.65 100.3) (end 192.65 108.8) (width 0.2) (layer "F.Cu") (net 7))
 (segment (start 187.25 94.9) (end 192.65 100.3) (width 0.2) (layer "F.Cu") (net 7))
 (segment (start 164.8 88.1) (end 164.8 72.2) (width 0.2) (layer "F.Cu") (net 7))
 (segment (start 176.2 94.9) (end 187.25 94.9) (width 0.2) (layer "F.Cu") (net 7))
 (segment (start 171.6 94.9) (end 164.8 88.1) (width 0.2) (layer "F.Cu") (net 7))
 (via (at 176.2 94.9) (size 0.6) (drill 0.3) (layers "F.Cu" "B.Cu") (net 7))
 (via (at 164.8 72.2) (size 0.6) (drill 0.3) (layers "F.Cu" "B.Cu") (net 7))
 (via (at 171.6 94.9) (size 0.6) (drill 0.3) (layers "F.Cu" "B.Cu") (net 7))
 (segment (start 163.7 71.1) (end 163.7 57.89) (width 0.2) (layer "B.Cu") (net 7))
 (segment (start 163.7 57.89) (end 165.15 56.44) (width 0.2) (layer "B.Cu") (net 7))
 (segment (start 164.8 72.2) (end 163.7 71.1) (width 0.2) (layer "B.Cu") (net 7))
 (segment (start 176.2 94.9) (end 171.6 94.9) (width 0.2) (layer "B.Cu") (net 7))
 (segment (start 204.35 111.6) (end 205.85 110.1) (width 0.2) (layer "F.Cu") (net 8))
 (segment (start 156.5 62) (end 159.52 58.98) (width 0.2) (layer "F.Cu") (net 8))
 (segment (start 151.14 74.26) (end 154.8 70.6) (width 0.2) (layer "F.Cu") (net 8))
 (segment (start 159.52 58.98) (end 165.15 58.98) (width 0.2) (layer "F.Cu") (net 8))
 (segment (start 175.592944 111.6) (end 151.14 87.147056) (width 0.2) (layer "F.Cu") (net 8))
 (segment (start 151.14 87.147056) (end 151.14 74.26) (width 0.2) (layer "F.Cu") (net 8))
 (segment (start 175.592944 111.6) (end 204.35 111.6) (width 0.2) (layer "F.Cu") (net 8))
 (via (at 156.5 62) (size 0.6) (drill 0.3) (layers "F.Cu" "B.Cu") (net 8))
 (via (at 154.8 70.6) (size 0.6) (drill 0.3) (layers "F.Cu" "B.Cu") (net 8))
 (segment (start 155.01 70.39) (end 155.01 63.49) (width 0.2) (layer "B.Cu") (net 8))
 (segment (start 154.8 70.6) (end 155.01 70.39) (width 0.2) (layer "B.Cu") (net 8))
 (segment (start 155.01 63.49) (end 156.5 62) (width 0.2) (layer "B.Cu") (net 8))
 (segment (start 153.61 64.02) (end 162.65 64.02) (width 0.2) (layer "F.Cu") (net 3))
 (segment (start 162.65 64.02) (end 165.15 61.52) (width 0.2) (layer "F.Cu") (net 3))
 (segment (start 153.61 80.68) (end 165.15 69.14) (width 0.2) (layer "F.Cu") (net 2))
 (segment (start 153.61 83.11) (end 153.61 80.68) (width 0.2) (layer "F.Cu") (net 2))
 (segment (start 149.9 98.49) (end 149.9 69.14) (width 0.2) (layer "F.Cu") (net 4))
 (segment (start 153.61 102.2) (end 149.9 98.49) (width 0.2) (layer "F.Cu") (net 4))
 (segment (start 173.87 64.06) (end 172.72 65.21) (width 0.2) (layer "F.Cu") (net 9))
 (segment (start 152.21 68.91) (end 149.9 66.6) (width 0.2) (layer "F.Cu") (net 9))
 (segment (start 158.393402 68.91) (end 152.21 68.91) (width 0.2) (layer "F.Cu") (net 9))
 (segment (start 172.72 65.21) (end 162.093402 65.21) (width 0.2) (layer "F.Cu") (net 9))
 (segment (start 162.093402 65.21) (end 158.393402 68.91) (width 0.2) (layer "F.Cu") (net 9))
 (segment (start 161.653553 63.440101) (end 155.01 63.440101) (width 0.2) (layer "F.Cu") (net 5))
 (segment (start 155.01 63.440101) (end 154.189899 62.62) (width 0.2) (layer "F.Cu") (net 5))
 (segment (start 175.27 81.75) (end 175.27 63.480101) (width 0.2) (layer "F.Cu") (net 5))
 (segment (start 175.27 63.480101) (end 172.159899 60.37) (width 0.2) (layer "F.Cu") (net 5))
 (segment (start 151.34 62.62) (end 149.9 64.06) (width 0.2) (layer "F.Cu") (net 5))
 (segment (start 154.189899 62.62) (end 151.34 62.62) (width 0.2) (layer "F.Cu") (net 5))
 (segment (start 164.723654 60.37) (end 161.653553 63.440101) (width 0.2) (layer "F.Cu") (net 5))
 (segment (start 173.87 83.15) (end 175.27 81.75) (width 0.2) (layer "F.Cu") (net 5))
 (segment (start 172.159899 60.37) (end 164.723654 60.37) (width 0.2) (layer "F.Cu") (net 5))
 (segment (start 174.103402 59.7) (end 168.4 59.7) (width 0.2) (layer "F.Cu") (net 10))
 (segment (start 153.59 57.83) (end 149.9 61.52) (width 0.2) (layer "F.Cu") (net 10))
 (segment (start 173.8 102.17) (end 173.8 86.199899) (width 0.2) (layer "F.Cu") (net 10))
 (segment (start 173.8 86.199899) (end 178.653402 81.346497) (width 0.2) (layer "F.Cu") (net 10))
 (segment (start 178.653402 81.346497) (end 178.653402 68.95) (width 0.2) (layer "F.Cu") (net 10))
 (segment (start 180.03 67.573402) (end 180.03 65.626598) (width 0.2) (layer "F.Cu") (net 10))
 (segment (start 180.03 65.626598) (end 174.103402 59.7) (width 0.2) (layer "F.Cu") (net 10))
 (segment (start 173.87 102.24) (end 173.8 102.17) (width 0.2) (layer "F.Cu") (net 10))
 (segment (start 168.4 59.7) (end 168.4 58.653654) (width 0.2) (layer "F.Cu") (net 10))
 (segment (start 168.4 58.653654) (end 167.576346 57.83) (width 0.2) (layer "F.Cu") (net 10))
 (segment (start 167.576346 57.83) (end 153.59 57.83) (width 0.2) (layer "F.Cu") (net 10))
 (segment (start 178.653402 68.95) (end 180.03 67.573402) (width 0.2) (layer "F.Cu") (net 10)))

